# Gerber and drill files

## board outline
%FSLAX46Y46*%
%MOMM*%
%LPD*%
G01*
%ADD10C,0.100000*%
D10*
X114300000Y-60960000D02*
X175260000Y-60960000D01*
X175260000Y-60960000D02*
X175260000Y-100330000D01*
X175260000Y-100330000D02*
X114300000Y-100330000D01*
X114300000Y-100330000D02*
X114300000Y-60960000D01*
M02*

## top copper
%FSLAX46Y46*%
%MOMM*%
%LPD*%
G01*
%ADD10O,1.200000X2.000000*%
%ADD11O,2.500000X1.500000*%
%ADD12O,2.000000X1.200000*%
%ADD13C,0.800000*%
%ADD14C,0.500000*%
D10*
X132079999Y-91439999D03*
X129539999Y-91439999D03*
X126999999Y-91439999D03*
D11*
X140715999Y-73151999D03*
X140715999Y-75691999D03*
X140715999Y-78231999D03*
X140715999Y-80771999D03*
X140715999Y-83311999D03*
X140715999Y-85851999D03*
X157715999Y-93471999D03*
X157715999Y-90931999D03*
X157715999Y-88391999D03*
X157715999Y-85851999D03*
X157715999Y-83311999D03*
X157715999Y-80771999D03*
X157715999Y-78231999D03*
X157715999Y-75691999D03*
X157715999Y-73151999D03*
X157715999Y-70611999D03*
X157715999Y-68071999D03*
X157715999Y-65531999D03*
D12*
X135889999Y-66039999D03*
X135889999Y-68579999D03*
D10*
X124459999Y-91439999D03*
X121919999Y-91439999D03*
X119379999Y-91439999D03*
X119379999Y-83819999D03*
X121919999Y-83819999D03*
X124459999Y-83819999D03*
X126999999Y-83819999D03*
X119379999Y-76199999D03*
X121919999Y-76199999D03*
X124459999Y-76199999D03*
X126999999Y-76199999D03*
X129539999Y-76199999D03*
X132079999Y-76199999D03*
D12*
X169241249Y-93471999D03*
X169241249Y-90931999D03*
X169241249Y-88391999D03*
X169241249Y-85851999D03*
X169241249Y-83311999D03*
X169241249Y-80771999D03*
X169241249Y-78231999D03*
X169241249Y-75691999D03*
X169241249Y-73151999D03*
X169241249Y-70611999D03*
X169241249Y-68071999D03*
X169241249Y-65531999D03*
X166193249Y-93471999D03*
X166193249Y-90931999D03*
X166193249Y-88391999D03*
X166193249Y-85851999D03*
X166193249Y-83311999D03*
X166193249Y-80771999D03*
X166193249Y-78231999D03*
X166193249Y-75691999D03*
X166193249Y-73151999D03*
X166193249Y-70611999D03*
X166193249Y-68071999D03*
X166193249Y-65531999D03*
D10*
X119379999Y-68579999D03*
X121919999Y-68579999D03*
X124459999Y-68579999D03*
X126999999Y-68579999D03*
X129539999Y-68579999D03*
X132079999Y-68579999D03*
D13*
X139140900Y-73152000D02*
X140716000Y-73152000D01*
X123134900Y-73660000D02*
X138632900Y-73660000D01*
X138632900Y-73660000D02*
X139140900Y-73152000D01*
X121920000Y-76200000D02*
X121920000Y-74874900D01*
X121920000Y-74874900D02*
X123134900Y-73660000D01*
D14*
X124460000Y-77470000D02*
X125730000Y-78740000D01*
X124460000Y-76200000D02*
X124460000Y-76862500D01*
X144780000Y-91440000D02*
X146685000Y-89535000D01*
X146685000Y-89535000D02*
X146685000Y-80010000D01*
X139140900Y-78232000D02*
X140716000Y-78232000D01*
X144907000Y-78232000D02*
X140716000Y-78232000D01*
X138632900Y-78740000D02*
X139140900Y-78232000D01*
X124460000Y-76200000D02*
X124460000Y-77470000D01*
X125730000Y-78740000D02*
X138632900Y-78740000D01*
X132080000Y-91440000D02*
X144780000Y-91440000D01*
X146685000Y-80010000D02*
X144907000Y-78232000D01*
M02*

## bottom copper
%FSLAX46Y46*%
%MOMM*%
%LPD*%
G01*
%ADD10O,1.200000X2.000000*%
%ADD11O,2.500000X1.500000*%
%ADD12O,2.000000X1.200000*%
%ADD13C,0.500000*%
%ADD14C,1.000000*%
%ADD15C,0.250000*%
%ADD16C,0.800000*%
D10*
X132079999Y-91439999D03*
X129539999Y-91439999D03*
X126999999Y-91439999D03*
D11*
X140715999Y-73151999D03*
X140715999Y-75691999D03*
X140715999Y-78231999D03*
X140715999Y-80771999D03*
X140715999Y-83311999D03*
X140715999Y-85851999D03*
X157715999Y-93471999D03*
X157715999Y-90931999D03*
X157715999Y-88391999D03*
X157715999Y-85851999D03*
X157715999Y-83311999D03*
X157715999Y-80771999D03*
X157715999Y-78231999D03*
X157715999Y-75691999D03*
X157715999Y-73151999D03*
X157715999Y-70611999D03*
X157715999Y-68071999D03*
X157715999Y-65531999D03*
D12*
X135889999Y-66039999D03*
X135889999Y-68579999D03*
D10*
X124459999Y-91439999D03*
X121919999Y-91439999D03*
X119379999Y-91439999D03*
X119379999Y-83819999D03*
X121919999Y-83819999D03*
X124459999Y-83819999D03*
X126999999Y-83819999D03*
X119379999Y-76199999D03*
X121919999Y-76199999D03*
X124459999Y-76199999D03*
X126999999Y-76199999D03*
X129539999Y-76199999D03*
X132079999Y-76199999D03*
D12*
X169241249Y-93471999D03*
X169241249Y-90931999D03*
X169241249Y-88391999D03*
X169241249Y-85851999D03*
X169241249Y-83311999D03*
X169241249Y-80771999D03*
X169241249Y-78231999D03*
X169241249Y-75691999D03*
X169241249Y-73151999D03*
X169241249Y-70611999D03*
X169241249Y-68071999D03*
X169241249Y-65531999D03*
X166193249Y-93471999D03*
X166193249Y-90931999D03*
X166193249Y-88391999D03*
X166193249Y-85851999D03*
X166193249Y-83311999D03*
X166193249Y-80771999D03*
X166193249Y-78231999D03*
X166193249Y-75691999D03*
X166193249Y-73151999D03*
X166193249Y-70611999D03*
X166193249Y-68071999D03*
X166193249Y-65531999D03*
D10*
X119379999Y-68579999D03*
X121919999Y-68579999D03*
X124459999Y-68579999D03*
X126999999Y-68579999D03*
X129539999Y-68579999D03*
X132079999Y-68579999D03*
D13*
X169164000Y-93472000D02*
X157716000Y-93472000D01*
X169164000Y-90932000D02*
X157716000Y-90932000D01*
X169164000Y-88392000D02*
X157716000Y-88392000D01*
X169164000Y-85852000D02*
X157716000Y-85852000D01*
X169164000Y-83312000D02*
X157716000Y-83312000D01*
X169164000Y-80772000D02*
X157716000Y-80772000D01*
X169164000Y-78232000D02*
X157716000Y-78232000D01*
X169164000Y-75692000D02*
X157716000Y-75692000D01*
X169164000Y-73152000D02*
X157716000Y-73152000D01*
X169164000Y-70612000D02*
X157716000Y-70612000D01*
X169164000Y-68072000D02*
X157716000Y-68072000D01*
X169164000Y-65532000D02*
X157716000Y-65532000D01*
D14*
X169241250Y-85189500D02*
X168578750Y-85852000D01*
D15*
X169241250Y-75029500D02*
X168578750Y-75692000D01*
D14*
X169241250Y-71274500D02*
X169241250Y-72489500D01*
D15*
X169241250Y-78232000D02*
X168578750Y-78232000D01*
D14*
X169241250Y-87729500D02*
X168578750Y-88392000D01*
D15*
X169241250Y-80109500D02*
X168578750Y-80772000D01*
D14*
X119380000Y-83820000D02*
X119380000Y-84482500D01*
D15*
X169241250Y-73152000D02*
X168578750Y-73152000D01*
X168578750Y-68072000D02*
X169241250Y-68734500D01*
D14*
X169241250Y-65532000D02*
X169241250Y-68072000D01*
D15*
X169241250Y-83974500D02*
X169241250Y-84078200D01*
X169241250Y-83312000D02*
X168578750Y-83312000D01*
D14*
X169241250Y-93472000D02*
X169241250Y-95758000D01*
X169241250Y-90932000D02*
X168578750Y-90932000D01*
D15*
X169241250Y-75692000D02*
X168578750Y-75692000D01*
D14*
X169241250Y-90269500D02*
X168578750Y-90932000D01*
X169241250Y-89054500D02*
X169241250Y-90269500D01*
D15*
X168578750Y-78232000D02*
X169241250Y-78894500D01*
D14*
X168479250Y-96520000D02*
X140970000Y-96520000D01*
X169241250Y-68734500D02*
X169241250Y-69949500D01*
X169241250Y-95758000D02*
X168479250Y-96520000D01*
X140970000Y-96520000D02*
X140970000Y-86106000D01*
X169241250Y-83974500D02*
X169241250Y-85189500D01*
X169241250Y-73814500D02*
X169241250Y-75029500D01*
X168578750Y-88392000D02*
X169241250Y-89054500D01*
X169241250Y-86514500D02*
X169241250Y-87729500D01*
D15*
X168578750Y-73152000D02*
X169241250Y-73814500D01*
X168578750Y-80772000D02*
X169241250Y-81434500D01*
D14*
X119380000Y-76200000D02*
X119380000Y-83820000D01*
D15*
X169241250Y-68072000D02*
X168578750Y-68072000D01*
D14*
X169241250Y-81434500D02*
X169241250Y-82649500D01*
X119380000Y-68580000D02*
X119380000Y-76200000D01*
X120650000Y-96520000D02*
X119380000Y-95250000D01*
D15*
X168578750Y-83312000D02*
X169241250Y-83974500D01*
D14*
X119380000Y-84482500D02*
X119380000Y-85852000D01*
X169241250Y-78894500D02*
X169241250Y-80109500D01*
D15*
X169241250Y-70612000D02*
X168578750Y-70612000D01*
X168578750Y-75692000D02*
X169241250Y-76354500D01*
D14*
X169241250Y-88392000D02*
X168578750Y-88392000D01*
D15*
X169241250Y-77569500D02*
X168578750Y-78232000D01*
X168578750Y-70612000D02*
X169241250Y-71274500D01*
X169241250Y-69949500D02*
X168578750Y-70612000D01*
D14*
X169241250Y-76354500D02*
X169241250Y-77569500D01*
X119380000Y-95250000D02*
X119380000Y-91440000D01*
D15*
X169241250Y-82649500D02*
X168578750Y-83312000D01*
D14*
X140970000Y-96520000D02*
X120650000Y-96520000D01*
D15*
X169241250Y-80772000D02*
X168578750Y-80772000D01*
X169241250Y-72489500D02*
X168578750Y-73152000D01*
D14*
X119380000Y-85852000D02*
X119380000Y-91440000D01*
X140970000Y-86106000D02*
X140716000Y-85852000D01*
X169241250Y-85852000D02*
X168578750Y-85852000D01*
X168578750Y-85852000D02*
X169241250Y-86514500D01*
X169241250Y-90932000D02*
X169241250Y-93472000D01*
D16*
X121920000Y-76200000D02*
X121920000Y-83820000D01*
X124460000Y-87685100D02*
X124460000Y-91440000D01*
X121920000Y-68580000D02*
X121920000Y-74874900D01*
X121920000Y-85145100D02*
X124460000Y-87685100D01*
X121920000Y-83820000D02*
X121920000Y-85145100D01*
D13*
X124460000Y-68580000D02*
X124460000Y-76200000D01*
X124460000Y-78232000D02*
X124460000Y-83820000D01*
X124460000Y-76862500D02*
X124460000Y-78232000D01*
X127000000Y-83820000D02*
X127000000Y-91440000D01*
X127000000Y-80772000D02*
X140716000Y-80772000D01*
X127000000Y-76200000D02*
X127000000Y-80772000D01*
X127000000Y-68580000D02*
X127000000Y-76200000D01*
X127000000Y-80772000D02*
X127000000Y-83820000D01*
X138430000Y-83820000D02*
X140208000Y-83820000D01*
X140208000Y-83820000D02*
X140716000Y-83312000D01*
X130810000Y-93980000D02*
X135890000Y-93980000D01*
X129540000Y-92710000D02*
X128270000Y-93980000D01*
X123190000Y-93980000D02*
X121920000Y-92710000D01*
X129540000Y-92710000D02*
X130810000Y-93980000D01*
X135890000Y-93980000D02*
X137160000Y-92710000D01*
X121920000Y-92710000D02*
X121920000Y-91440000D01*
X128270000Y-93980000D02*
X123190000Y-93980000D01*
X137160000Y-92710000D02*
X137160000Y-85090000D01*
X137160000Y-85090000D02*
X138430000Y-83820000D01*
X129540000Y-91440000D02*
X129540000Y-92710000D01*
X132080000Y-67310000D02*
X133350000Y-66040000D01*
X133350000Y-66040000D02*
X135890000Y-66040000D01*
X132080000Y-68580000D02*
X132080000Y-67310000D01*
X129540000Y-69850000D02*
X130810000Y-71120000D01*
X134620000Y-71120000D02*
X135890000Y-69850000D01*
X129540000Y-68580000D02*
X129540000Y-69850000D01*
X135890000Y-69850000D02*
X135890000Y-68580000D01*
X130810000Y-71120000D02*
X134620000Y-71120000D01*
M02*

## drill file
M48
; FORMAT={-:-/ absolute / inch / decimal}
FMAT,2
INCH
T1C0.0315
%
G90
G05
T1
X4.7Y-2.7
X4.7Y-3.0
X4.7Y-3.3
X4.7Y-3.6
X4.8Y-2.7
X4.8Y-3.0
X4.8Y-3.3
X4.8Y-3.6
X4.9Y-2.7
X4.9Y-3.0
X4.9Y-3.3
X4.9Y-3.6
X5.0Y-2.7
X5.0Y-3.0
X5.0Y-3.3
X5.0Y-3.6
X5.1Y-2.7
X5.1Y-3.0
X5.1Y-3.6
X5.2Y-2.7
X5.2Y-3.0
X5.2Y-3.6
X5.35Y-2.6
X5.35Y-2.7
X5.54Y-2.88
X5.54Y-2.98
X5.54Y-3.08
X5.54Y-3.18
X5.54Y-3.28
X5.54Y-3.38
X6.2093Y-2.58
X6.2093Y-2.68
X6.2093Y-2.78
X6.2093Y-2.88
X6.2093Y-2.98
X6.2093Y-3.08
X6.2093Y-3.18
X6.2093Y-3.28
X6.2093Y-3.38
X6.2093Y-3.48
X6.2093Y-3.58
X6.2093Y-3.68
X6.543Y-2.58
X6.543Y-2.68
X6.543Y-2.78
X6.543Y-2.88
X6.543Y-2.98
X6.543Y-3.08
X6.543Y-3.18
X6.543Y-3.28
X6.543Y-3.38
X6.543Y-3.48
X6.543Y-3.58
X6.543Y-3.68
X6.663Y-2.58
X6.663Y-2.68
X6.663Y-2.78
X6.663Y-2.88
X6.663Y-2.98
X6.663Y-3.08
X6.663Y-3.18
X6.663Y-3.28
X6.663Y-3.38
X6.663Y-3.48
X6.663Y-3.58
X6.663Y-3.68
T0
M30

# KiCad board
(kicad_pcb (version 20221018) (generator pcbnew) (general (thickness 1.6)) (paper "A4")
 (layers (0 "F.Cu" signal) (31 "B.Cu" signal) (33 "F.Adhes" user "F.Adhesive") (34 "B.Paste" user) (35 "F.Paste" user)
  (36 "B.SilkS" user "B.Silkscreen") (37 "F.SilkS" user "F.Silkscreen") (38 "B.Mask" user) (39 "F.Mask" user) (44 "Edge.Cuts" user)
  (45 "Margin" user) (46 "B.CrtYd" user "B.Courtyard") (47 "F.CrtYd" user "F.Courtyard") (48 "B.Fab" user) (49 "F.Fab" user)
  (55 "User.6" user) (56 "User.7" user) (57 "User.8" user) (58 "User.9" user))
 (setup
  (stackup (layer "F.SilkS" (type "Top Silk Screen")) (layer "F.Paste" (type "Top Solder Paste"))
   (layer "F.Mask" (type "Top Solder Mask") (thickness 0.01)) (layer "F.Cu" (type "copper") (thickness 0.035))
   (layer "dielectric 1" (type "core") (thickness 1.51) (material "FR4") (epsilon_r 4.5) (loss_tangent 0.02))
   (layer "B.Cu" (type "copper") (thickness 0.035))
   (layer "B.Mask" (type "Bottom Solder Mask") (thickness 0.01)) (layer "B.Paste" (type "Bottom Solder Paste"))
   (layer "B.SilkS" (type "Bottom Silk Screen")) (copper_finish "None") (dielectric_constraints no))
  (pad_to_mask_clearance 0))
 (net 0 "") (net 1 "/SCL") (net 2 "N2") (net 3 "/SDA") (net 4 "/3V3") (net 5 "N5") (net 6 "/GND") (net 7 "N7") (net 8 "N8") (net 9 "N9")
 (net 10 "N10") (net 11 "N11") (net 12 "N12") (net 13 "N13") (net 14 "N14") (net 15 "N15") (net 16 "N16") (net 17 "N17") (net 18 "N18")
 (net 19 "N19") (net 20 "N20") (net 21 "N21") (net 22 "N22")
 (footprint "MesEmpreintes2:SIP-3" (layer "F.Cu") (at 129.54 91.44 180)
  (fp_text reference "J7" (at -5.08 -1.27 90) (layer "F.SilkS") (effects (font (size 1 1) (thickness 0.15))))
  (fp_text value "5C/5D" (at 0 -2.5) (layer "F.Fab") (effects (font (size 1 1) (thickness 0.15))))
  (pad "1" thru_hole oval (at -2.54 0 180) (size 1.2 2) (drill 0.8) (layers "*.Cu" "*.Mask") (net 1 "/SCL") (thermal_bridge_angle 45))
  (pad "2" thru_hole oval (at 0 0 180) (size 1.2 2) (drill 0.8) (layers "*.Cu" "*.Mask") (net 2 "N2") (thermal_bridge_angle 45))
  (pad "3" thru_hole oval (at 2.54 0 180) (size 1.2 2) (drill 0.8) (layers "*.Cu" "*.Mask") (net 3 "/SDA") (thermal_bridge_angle 45)))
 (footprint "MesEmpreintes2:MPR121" (layer "F.Cu") (at 149.216 79.502 -90)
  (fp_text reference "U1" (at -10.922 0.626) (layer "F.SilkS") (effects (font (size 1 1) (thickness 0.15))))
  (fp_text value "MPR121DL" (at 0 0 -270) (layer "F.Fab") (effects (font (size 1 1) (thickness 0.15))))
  (pad "1" thru_hole oval (at -6.35 8.5 270) (size 1.5 2.5) (drill 0.8) (layers "*.Cu" "*.Mask") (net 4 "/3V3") (thermal_bridge_angle 45))
  (pad "2" thru_hole oval (at -3.81 8.5 270) (size 1.5 2.5) (drill 0.8) (layers "*.Cu" "*.Mask") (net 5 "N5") (thermal_bridge_angle 45))
  (pad "3" thru_hole oval (at -1.27 8.5 270) (size 1.5 2.5) (drill 0.8) (layers "*.Cu" "*.Mask") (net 1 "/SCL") (thermal_bridge_angle 45))
  (pad "4" thru_hole oval (at 1.27 8.5 270) (size 1.5 2.5) (drill 0.8) (layers "*.Cu" "*.Mask") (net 3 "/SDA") (thermal_bridge_angle 45))
  (pad "5" thru_hole oval (at 3.81 8.5 270) (size 1.5 2.5) (drill 0.8) (layers "*.Cu" "*.Mask") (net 2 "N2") (thermal_bridge_angle 45))
  (pad "6" thru_hole oval (at 6.35 8.5 270) (size 1.5 2.5) (drill 0.8) (layers "*.Cu" "*.Mask") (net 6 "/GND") (thermal_bridge_angle 45))
  (pad "7" thru_hole oval (at 13.97 -8.5 270) (size 1.5 2.5) (drill 0.8) (layers "*.Cu" "*.Mask") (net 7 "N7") (thermal_bridge_angle 45))
  (pad "8" thru_hole oval (at 11.43 -8.5 270) (size 1.5 2.5) (drill 0.8) (layers "*.Cu" "*.Mask") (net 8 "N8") (thermal_bridge_angle 45))
  (pad "9" thru_hole oval (at 8.89 -8.5 270) (size 1.5 2.5) (drill 0.8) (layers "*.Cu" "*.Mask") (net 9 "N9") (thermal_bridge_angle 45))
  (pad "10" thru_hole oval (at 6.35 -8.5 270) (size 1.5 2.5) (drill 0.8) (layers "*.Cu" "*.Mask") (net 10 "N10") (thermal_bridge_angle 45))
  (pad "11" thru_hole oval (at 3.81 -8.5 270) (size 1.5 2.5) (drill 0.8) (layers "*.Cu" "*.Mask") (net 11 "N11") (thermal_bridge_angle 45))
  (pad "12" thru_hole oval (at 1.27 -8.5 270) (size 1.5 2.5) (drill 0.8) (layers "*.Cu" "*.Mask") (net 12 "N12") (thermal_bridge_angle 45))
  (pad "13" thru_hole oval (at -1.27 -8.5 270) (size 1.5 2.5) (drill 0.8) (layers "*.Cu" "*.Mask") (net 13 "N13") (thermal_bridge_angle 45))
  (pad "14" thru_hole oval (at -3.81 -8.5 270) (size 1.5 2.5) (drill 0.8) (layers "*.Cu" "*.Mask") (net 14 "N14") (thermal_bridge_angle 45))
  (pad "15" thru_hole oval (at -6.35 -8.5 270) (size 1.5 2.5) (drill 0.8) (layers "*.Cu" "*.Mask") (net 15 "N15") (thermal_bridge_angle 45))
  (pad "16" thru_hole oval (at -8.89 -8.5 270) (size 1.5 2.5) (drill 0.8) (layers "*.Cu" "*.Mask") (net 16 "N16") (thermal_bridge_angle 45))
  (pad "17" thru_hole oval (at -11.43 -8.5 270) (size 1.5 2.5) (drill 0.8) (layers "*.Cu" "*.Mask") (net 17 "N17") (thermal_bridge_angle 45))
  (pad "18" thru_hole oval (at -13.97 -8.5 270) (size 1.5 2.5) (drill 0.8) (layers "*.Cu" "*.Mask") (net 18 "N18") (thermal_bridge_angle 45)))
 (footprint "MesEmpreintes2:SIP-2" (layer "F.Cu") (at 135.89 67.31 -90)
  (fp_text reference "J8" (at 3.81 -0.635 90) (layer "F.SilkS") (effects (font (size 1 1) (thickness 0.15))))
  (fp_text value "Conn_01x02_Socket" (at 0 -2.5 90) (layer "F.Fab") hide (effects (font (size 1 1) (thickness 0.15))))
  (pad "1" thru_hole oval (at -1.27 0 270) (size 1.2 2) (drill 0.8) (layers "*.Cu" "*.Mask") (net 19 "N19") (thermal_bridge_angle 45))
  (pad "2" thru_hole oval (at 1.27 0 270) (size 1.2 2) (drill 0.8) (layers "*.Cu" "*.Mask") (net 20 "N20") (thermal_bridge_angle 45)))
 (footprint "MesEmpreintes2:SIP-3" (layer "F.Cu") (at 121.92 91.44 180)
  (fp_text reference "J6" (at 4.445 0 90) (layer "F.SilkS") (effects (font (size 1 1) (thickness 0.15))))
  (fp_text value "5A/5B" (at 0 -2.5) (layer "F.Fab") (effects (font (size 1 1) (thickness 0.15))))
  (pad "1" thru_hole oval (at -2.54 0 180) (size 1.2 2) (drill 0.8) (layers "*.Cu" "*.Mask") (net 4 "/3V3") (thermal_bridge_angle 45))
  (pad "2" thru_hole oval (at 0 0 180) (size 1.2 2) (drill 0.8) (layers "*.Cu" "*.Mask") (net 2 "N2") (thermal_bridge_angle 45))
  (pad "3" thru_hole oval (at 2.54 0 180) (size 1.2 2) (drill 0.8) (layers "*.Cu" "*.Mask") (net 6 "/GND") (thermal_bridge_angle 45)))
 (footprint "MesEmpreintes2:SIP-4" (layer "F.Cu") (at 123.19 83.82)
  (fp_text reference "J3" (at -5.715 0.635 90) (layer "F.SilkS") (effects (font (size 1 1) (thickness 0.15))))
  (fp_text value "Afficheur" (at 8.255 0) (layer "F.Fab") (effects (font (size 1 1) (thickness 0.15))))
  (pad "1" thru_hole oval (at -3.81 0) (size 1.2 2) (drill 0.8) (layers "*.Cu" "*.Mask") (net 6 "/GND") (thermal_bridge_angle 45))
  (pad "2" thru_hole oval (at -1.27 0) (size 1.2 2) (drill 0.8) (layers "*.Cu" "*.Mask") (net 4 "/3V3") (thermal_bridge_angle 45))
  (pad "3" thru_hole oval (at 1.27 0) (size 1.2 2) (drill 0.8) (layers "*.Cu" "*.Mask") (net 1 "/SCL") (thermal_bridge_angle 45))
  (pad "4" thru_hole oval (at 3.81 0) (size 1.2 2) (drill 0.8) (layers "*.Cu" "*.Mask") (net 3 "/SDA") (thermal_bridge_angle 45)))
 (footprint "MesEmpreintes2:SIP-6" (layer "F.Cu") (at 125.73 76.2)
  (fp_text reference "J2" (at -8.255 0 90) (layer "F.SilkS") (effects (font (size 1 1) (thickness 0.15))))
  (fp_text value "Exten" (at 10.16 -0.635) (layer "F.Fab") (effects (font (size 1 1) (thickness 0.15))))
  (pad "1" thru_hole oval (at -6.35 0) (size 1.2 2) (drill 0.8) (layers "*.Cu" "*.Mask") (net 6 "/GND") (thermal_bridge_angle 45))
  (pad "2" thru_hole oval (at -3.81 0) (size 1.2 2) (drill 0.8) (layers "*.Cu" "*.Mask") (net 4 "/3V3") (thermal_bridge_angle 45))
  (pad "3" thru_hole oval (at -1.27 0) (size 1.2 2) (drill 0.8) (layers "*.Cu" "*.Mask") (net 1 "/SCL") (thermal_bridge_angle 45))
  (pad "4" thru_hole oval (at 1.27 0) (size 1.2 2) (drill 0.8) (layers "*.Cu" "*.Mask") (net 3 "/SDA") (thermal_bridge_angle 45))
  (pad "5" thru_hole oval (at 3.81 0) (size 1.2 2) (drill 0.8) (layers "*.Cu" "*.Mask") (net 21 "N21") (thermal_bridge_angle 45))
  (pad "6" thru_hole oval (at 6.35 0) (size 1.2 2) (drill 0.8) (layers "*.Cu" "*.Mask") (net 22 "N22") (thermal_bridge_angle 45)))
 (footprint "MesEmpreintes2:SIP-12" (layer "F.Cu") (at 169.24125 79.502 90)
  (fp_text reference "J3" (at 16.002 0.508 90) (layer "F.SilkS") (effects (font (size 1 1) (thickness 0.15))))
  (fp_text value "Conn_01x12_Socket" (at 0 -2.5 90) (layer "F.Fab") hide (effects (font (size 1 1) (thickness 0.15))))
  (pad "1" thru_hole oval (at -13.97 0 90) (size 1.2 2) (drill 0.8) (layers "*.Cu" "*.Mask") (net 6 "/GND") (thermal_bridge_angle 45))
  (pad "2" thru_hole oval (at -11.43 0 90) (size 1.2 2) (drill 0.8) (layers "*.Cu" "*.Mask") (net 6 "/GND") (thermal_bridge_angle 45))
  (pad "3" thru_hole oval (at -8.89 0 90) (size 1.2 2) (drill 0.8) (layers "*.Cu" "*.Mask") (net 6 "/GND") (thermal_bridge_angle 45))
  (pad "4" thru_hole oval (at -6.35 0 90) (size 1.2 2) (drill 0.8) (layers "*.Cu" "*.Mask") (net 6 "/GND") (thermal_bridge_angle 45))
  (pad "5" thru_hole oval (at -3.81 0 90) (size 1.2 2) (drill 0.8) (layers "*.Cu" "*.Mask") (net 6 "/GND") (thermal_bridge_angle 45))
  (pad "6" thru_hole oval (at -1.27 0 90) (size 1.2 2) (drill 0.8) (layers "*.Cu" "*.Mask") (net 6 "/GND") (thermal_bridge_angle 45))
  (pad "7" thru_hole oval (at 1.27 0 90) (size 1.2 2) (drill 0.8) (layers "*.Cu" "*.Mask") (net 6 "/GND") (thermal_bridge_angle 45))
  (pad "8" thru_hole oval (at 3.81 0 90) (size 1.2 2) (drill 0.8) (layers "*.Cu" "*.Mask") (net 6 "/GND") (thermal_bridge_angle 45))
  (pad "9" thru_hole oval (at 6.35 0 90) (size 1.2 2) (drill 0.8) (layers "*.Cu" "*.Mask") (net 6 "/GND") (thermal_bridge_angle 45))
  (pad "10" thru_hole oval (at 8.89 0 90) (size 1.2 2) (drill 0.8) (layers "*.Cu" "*.Mask") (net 6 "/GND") (thermal_bridge_angle 45))
  (pad "11" thru_hole oval (at 11.43 0 90) (size 1.2 2) (drill 0.8) (layers "*.Cu" "*.Mask") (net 6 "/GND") (thermal_bridge_angle 45))
  (pad "12" thru_hole oval (at 13.97 0 90) (size 1.2 2) (drill 0.8) (layers "*.Cu" "*.Mask") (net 6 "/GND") (thermal_bridge_angle 45)))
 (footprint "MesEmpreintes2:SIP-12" (layer "F.Cu") (at 166.19325 79.502 90)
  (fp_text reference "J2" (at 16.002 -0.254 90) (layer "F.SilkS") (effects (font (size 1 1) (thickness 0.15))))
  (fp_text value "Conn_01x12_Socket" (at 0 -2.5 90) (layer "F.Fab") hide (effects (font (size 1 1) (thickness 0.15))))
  (pad "1" thru_hole oval (at -13.97 0 90) (size 1.2 2) (drill 0.8) (layers "*.Cu" "*.Mask") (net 7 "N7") (thermal_bridge_angle 45))
  (pad "2" thru_hole oval (at -11.43 0 90) (size 1.2 2) (drill 0.8) (layers "*.Cu" "*.Mask") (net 8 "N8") (thermal_bridge_angle 45))
  (pad "3" thru_hole oval (at -8.89 0 90) (size 1.2 2) (drill 0.8) (layers "*.Cu" "*.Mask") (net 9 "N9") (thermal_bridge_angle 45))
  (pad "4" thru_hole oval (at -6.35 0 90) (size 1.2 2) (drill 0.8) (layers "*.Cu" "*.Mask") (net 10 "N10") (thermal_bridge_angle 45))
  (pad "5" thru_hole oval (at -3.81 0 90) (size 1.2 2) (drill 0.8) (layers "*.Cu" "*.Mask") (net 11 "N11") (thermal_bridge_angle 45))
  (pad "6" thru_hole oval (at -1.27 0 90) (size 1.2 2) (drill 0.8) (layers "*.Cu" "*.Mask") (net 12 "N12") (thermal_bridge_angle 45))
  (pad "7" thru_hole oval (at 1.27 0 90) (size 1.2 2) (drill 0.8) (layers "*.Cu" "*.Mask") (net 13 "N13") (thermal_bridge_angle 45))
  (pad "8" thru_hole oval (at 3.81 0 90) (size 1.2 2) (drill 0.8) (layers "*.Cu" "*.Mask") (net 14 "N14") (thermal_bridge_angle 45))
  (pad "9" thru_hole oval (at 6.35 0 90) (size 1.2 2) (drill 0.8) (layers "*.Cu" "*.Mask") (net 15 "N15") (thermal_bridge_angle 45))
  (pad "10" thru_hole oval (at 8.89 0 90) (size 1.2 2) (drill 0.8) (layers "*.Cu" "*.Mask") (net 16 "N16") (thermal_bridge_angle 45))
  (pad "11" thru_hole oval (at 11.43 0 90) (size 1.2 2) (drill 0.8) (layers "*.Cu" "*.Mask") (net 17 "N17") (thermal_bridge_angle 45))
  (pad "12" thru_hole oval (at 13.97 0 90) (size 1.2 2) (drill 0.8) (layers "*.Cu" "*.Mask") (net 18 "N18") (thermal_bridge_angle 45)))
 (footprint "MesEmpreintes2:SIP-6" (layer "F.Cu") (at 125.73 68.58)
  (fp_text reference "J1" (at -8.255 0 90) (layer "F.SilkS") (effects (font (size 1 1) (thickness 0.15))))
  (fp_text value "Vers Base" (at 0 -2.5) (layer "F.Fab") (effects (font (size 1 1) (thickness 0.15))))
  (pad "1" thru_hole oval (at -6.35 0) (size 1.2 2) (drill 0.8) (layers "*.Cu" "*.Mask") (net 6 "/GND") (thermal_bridge_angle 45))
  (pad "2" thru_hole oval (at -3.81 0) (size 1.2 2) (drill 0.8) (layers "*.Cu" "*.Mask") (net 4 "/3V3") (thermal_bridge_angle 45))
  (pad "3" thru_hole oval (at -1.27 0) (size 1.2 2) (drill 0.8) (layers "*.Cu" "*.Mask") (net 1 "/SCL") (thermal_bridge_angle 45))
  (pad "4" thru_hole oval (at 1.27 0) (size 1.2 2) (drill 0.8) (layers "*.Cu" "*.Mask") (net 3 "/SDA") (thermal_bridge_angle 45))
  (pad "5" thru_hole oval (at 3.81 0) (size 1.2 2) (drill 0.8) (layers "*.Cu" "*.Mask") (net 20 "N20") (thermal_bridge_angle 45))
  (pad "6" thru_hole oval (at 6.35 0) (size 1.2 2) (drill 0.8) (layers "*.Cu" "*.Mask") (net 19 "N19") (thermal_bridge_angle 45)))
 (gr_rect (start 114.3 60.96) (end 175.26 100.33) (stroke (width 0.1) (type default)) (fill none) (layer "Edge.Cuts"))
 (segment (start 169.164 93.472) (end 157.716 93.472) (width 0.5) (layer "B.Cu") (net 7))
 (segment (start 169.164 90.932) (end 157.716 90.932) (width 0.5) (layer "B.Cu") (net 8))
 (segment (start 169.164 88.392) (end 157.716 88.392) (width 0.5) (layer "B.Cu") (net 9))
 (segment (start 169.164 85.852) (end 157.716 85.852) (width 0.5) (layer "B.Cu") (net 10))
 (segment (start 169.164 83.312) (end 157.716 83.312) (width 0.5) (layer "B.Cu") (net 11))
 (segment (start 169.164 80.772) (end 157.716 80.772) (width 0.5) (layer "B.Cu") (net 12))
 (segment (start 169.164 78.232) (end 157.716 78.232) (width 0.5) (layer "B.Cu") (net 13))
 (segment (start 169.164 75.692) (end 157.716 75.692) (width 0.5) (layer "B.Cu") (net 14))
 (segment (start 169.164 73.152) (end 157.716 73.152) (width 0.5) (layer "B.Cu") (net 15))
 (segment (start 169.164 70.612) (end 157.716 70.612) (width 0.5) (layer "B.Cu") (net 16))
 (segment (start 169.164 68.072) (end 157.716 68.072) (width 0.5) (layer "B.Cu") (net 17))
 (segment (start 169.164 65.532) (end 157.716 65.532) (width 0.5) (layer "B.Cu") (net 18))
 (segment (start 169.24125 85.1895) (end 168.57875 85.852) (width 1) (layer "B.Cu") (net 6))
 (segment (start 169.24125 75.0295) (end 168.57875 75.692) (width 0.25) (layer "B.Cu") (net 6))
 (segment (start 169.24125 71.2745) (end 169.24125 72.4895) (width 1) (layer "B.Cu") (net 6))
 (segment (start 169.24125 78.232) (end 168.57875 78.232) (width 0.25) (layer "B.Cu") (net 6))
 (segment (start 169.24125 87.7295) (end 168.57875 88.392) (width 1) (layer "B.Cu") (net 6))
 (segment (start 169.24125 80.1095) (end 168.57875 80.772) (width 0.25) (layer "B.Cu") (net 6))
 (segment (start 119.38 83.82) (end 119.38 84.4825) (width 1) (layer "B.Cu") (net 6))
 (segment (start 169.24125 73.152) (end 168.57875 73.152) (width 0.25) (layer "B.Cu") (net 6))
 (segment (start 168.57875 68.072) (end 169.24125 68.7345) (width 0.25) (layer "B.Cu") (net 6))
 (segment (start 169.24125 65.532) (end 169.24125 68.072) (width 1) (layer "B.Cu") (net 6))
 (segment (start 169.24125 83.9745) (end 169.24125 84.0782) (width 0.25) (layer "B.Cu") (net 6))
 (segment (start 169.24125 83.312) (end 168.57875 83.312) (width 0.25) (layer "B.Cu") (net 6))
 (segment (start 169.24125 93.472) (end 169.24125 95.758) (width 1) (layer "B.Cu") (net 6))
 (segment (start 169.24125 90.932) (end 168.57875 90.932) (width 1) (layer "B.Cu") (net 6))
 (segment (start 169.24125 75.692) (end 168.57875 75.692) (width 0.25) (layer "B.Cu") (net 6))
 (segment (start 169.24125 90.2695) (end 168.57875 90.932) (width 1) (layer "B.Cu") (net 6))
 (segment (start 169.24125 89.0545) (end 169.24125 90.2695) (width 1) (layer "B.Cu") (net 6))
 (segment (start 168.57875 78.232) (end 169.24125 78.8945) (width 0.25) (layer "B.Cu") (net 6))
 (segment (start 168.47925 96.52) (end 140.97 96.52) (width 1) (layer "B.Cu") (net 6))
 (segment (start 169.24125 68.7345) (end 169.24125 69.9495) (width 1) (layer "B.Cu") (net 6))
 (segment (start 169.24125 95.758) (end 168.47925 96.52) (width 1) (layer "B.Cu") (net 6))
 (segment (start 140.97 96.52) (end 140.97 86.106) (width 1) (layer "B.Cu") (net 6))
 (segment (start 169.24125 83.9745) (end 169.24125 85.1895) (width 1) (layer "B.Cu") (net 6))
 (segment (start 169.24125 73.8145) (end 169.24125 75.0295) (width 1) (layer "B.Cu") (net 6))
 (segment (start 168.57875 88.392) (end 169.24125 89.0545) (width 1) (layer "B.Cu") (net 6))
 (segment (start 169.24125 86.5145) (end 169.24125 87.7295) (width 1) (layer "B.Cu") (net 6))
 (segment (start 168.57875 73.152) (end 169.24125 73.8145) (width 0.25) (layer "B.Cu") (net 6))
 (segment (start 168.57875 80.772) (end 169.24125 81.4345) (width 0.25) (layer "B.Cu") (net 6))
 (segment (start 119.38 76.2) (end 119.38 83.82) (width 1) (layer "B.Cu") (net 6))
 (segment (start 169.24125 68.072) (end 168.57875 68.072) (width 0.25) (layer "B.Cu") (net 6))
 (segment (start 169.24125 81.4345) (end 169.24125 82.6495) (width 1) (layer "B.Cu") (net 6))
 (segment (start 119.38 68.58) (end 119.38 76.2) (width 1) (layer "B.Cu") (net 6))
 (segment (start 120.65 96.52) (end 119.38 95.25) (width 1) (layer "B.Cu") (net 6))
 (segment (start 168.57875 83.312) (end 169.24125 83.9745) (width 0.25) (layer "B.Cu") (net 6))
 (segment (start 119.38 84.4825) (end 119.38 85.852) (width 1) (layer "B.Cu") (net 6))
 (segment (start 169.24125 78.8945) (end 169.24125 80.1095) (width 1) (layer "B.Cu") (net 6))
 (segment (start 169.24125 70.612) (end 168.57875 70.612) (width 0.25) (layer "B.Cu") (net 6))
 (segment (start 168.57875 75.692) (end 169.24125 76.3545) (width 0.25) (layer "B.Cu") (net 6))
 (segment (start 169.24125 88.392) (end 168.57875 88.392) (width 1) (layer "B.Cu") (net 6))
 (segment (start 169.24125 77.5695) (end 168.57875 78.232) (width 0.25) (layer "B.Cu") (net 6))
 (segment (start 168.57875 70.612) (end 169.24125 71.2745) (width 0.25) (layer "B.Cu") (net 6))
 (segment (start 169.24125 69.9495) (end 168.57875 70.612) (width 0.25) (layer "B.Cu") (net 6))
 (segment (start 169.24125 76.3545) (end 169.24125 77.5695) (width 1) (layer "B.Cu") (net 6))
 (segment (start 119.38 95.25) (end 119.38 91.44) (width 1) (layer "B.Cu") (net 6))
 (segment (start 169.24125 82.6495) (end 168.57875 83.312) (width 0.25) (layer "B.Cu") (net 6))
 (segment (start 140.97 96.52) (end 120.65 96.52) (width 1) (layer "B.Cu") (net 6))
 (segment (start 169.24125 80.772) (end 168.57875 80.772) (width 0.25) (layer "B.Cu") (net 6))
 (segment (start 169.24125 72.4895) (end 168.57875 73.152) (width 0.25) (layer "B.Cu") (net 6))
 (segment (start 119.38 85.852) (end 119.38 91.44) (width 1) (layer "B.Cu") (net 6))
 (segment (start 140.97 86.106) (end 140.716 85.852) (width 1) (layer "B.Cu") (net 6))
 (segment (start 169.24125 85.852) (end 168.57875 85.852) (width 1) (layer "B.Cu") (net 6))
 (segment (start 168.57875 85.852) (end 169.24125 86.5145) (width 1) (layer "B.Cu") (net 6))
 (segment (start 169.24125 90.932) (end 169.24125 93.472) (width 1) (layer "B.Cu") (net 6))
 (segment (start 139.1409 73.152) (end 140.716 73.152) (width 0.8) (layer "F.Cu") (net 4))
 (segment (start 123.1349 73.66) (end 138.6329 73.66) (width 0.8) (layer "F.Cu") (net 4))
 (segment (start 138.6329 73.66) (end 139.1409 73.152) (width 0.8) (layer "F.Cu") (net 4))
 (segment (start 121.92 76.2) (end 121.92 74.8749) (width 0.8) (layer "F.Cu") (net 4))
 (segment (start 121.92 74.8749) (end 123.1349 73.66) (width 0.8) (layer "F.Cu") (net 4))
 (segment (start 121.92 76.2) (end 121.92 83.82) (width 0.8) (layer "B.Cu") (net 4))
 (segment (start 124.46 87.6851) (end 124.46 91.44) (width 0.8) (layer "B.Cu") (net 4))
 (segment (start 121.92 68.58) (end 121.92 74.8749) (width 0.8) (layer "B.Cu") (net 4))
 (segment (start 121.92 85.1451) (end 124.46 87.6851) (width 0.8) (layer "B.Cu") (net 4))
 (segment (start 121.92 83.82) (end 121.92 85.1451) (width 0.8) (layer "B.Cu") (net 4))
 (segment (start 124.46 77.47) (end 125.73 78.74) (width 0.5) (layer "F.Cu") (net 1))
 (segment (start 124.46 76.2) (end 124.46 76.8625) (width 0.5) (layer "F.Cu") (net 1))
 (segment (start 144.78 91.44) (end 146.685 89.535) (width 0.5) (layer "F.Cu") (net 1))
 (segment (start 146.685 89.535) (end 146.685 80.01) (width 0.5) (layer "F.Cu") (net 1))
 (segment (start 139.1409 78.232) (end 140.716 78.232) (width 0.5) (layer "F.Cu") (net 1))
 (segment (start 144.907 78.232) (end 140.716 78.232) (width 0.5) (layer "F.Cu") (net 1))
 (segment (start 138.6329 78.74) (end 139.1409 78.232) (width 0.5) (layer "F.Cu") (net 1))
 (segment (start 124.46 76.2) (end 124.46 77.47) (width 0.5) (layer "F.Cu") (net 1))
 (segment (start 125.73 78.74) (end 138.6329 78.74) (width 0.5) (layer "F.Cu") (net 1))
 (segment (start 132.08 91.44) (end 144.78 91.44) (width 0.5) (layer "F.Cu") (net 1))
 (segment (start 146.685 80.01) (end 144.907 78.232) (width 0.5) (layer "F.Cu") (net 1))
 (segment (start 124.46 68.58) (end 124.46 76.2) (width 0.5) (layer "B.Cu") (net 1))
 (segment (start 124.46 78.232) (end 124.46 83.82) (width 0.5) (layer "B.Cu") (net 1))
 (segment (start 124.46 76.8625) (end 124.46 78.232) (width 0.5) (layer "B.Cu") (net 1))
 (segment (start 127 83.82) (end 127 91.44) (width 0.5) (layer "B.Cu") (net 3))
 (segment (start 127 80.772) (end 140.716 80.772) (width 0.5) (layer "B.Cu") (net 3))
 (segment (start 127 76.2) (end 127 80.772) (width 0.5) (layer "B.Cu") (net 3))
 (segment (start 127 68.58) (end 127 76.2) (width 0.5) (layer "B.Cu") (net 3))
 (segment (start 127 80.772) (end 127 83.82) (width 0.5) (layer "B.Cu") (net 3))
 (segment (start 138.43 83.82) (end 140.208 83.82) (width 0.5) (layer "B.Cu") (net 2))
 (segment (start 140.208 83.82) (end 140.716 83.312) (width 0.5) (layer "B.Cu") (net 2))
 (segment (start 130.81 93.98) (end 135.89 93.98) (width 0.5) (layer "B.Cu") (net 2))
 (segment (start 129.54 92.71) (end 128.27 93.98) (width 0.5) (layer "B.Cu") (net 2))
 (segment (start 123.19 93.98) (end 121.92 92.71) (width 0.5) (layer "B.Cu") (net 2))
 (segment (start 129.54 92.71) (end 130.81 93.98) (width 0.5) (layer "B.Cu") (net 2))
 (segment (start 135.89 93.98) (end 137.16 92.71) (width 0.5) (layer "B.Cu") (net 2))
 (segment (start 121.92 92.71) (end 121.92 91.44) (width 0.5) (layer "B.Cu") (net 2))
 (segment (start 128.27 93.98) (end 123.19 93.98) (width 0.5) (layer "B.Cu") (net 2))
 (segment (start 137.16 92.71) (end 137.16 85.09) (width 0.5) (layer "B.Cu") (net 2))
 (segment (start 137.16 85.09) (end 138.43 83.82) (width 0.5) (layer "B.Cu") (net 2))
 (segment (start 129.54 91.44) (end 129.54 92.71) (width 0.5) (layer "B.Cu") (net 2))
 (segment (start 132.08 67.31) (end 133.35 66.04) (width 0.5) (layer "B.Cu") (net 19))
 (segment (start 133.35 66.04) (end 135.89 66.04) (width 0.5) (layer "B.Cu") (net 19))
 (segment (start 132.08 68.58) (end 132.08 67.31) (width 0.5) (layer "B.Cu") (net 19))
 (segment (start 129.54 69.85) (end 130.81 71.12) (width 0.5) (layer "B.Cu") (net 20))
 (segment (start 134.62 71.12) (end 135.89 69.85) (width 0.5) (layer "B.Cu") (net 20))
 (segment (start 129.54 68.58) (end 129.54 69.85) (width 0.5) (layer "B.Cu") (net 20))
 (segment (start 135.89 69.85) (end 135.89 68.58) (width 0.5) (layer "B.Cu") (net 20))
 (segment (start 130.81 71.12) (end 134.62 71.12) (width 0.5) (layer "B.Cu") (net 20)))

